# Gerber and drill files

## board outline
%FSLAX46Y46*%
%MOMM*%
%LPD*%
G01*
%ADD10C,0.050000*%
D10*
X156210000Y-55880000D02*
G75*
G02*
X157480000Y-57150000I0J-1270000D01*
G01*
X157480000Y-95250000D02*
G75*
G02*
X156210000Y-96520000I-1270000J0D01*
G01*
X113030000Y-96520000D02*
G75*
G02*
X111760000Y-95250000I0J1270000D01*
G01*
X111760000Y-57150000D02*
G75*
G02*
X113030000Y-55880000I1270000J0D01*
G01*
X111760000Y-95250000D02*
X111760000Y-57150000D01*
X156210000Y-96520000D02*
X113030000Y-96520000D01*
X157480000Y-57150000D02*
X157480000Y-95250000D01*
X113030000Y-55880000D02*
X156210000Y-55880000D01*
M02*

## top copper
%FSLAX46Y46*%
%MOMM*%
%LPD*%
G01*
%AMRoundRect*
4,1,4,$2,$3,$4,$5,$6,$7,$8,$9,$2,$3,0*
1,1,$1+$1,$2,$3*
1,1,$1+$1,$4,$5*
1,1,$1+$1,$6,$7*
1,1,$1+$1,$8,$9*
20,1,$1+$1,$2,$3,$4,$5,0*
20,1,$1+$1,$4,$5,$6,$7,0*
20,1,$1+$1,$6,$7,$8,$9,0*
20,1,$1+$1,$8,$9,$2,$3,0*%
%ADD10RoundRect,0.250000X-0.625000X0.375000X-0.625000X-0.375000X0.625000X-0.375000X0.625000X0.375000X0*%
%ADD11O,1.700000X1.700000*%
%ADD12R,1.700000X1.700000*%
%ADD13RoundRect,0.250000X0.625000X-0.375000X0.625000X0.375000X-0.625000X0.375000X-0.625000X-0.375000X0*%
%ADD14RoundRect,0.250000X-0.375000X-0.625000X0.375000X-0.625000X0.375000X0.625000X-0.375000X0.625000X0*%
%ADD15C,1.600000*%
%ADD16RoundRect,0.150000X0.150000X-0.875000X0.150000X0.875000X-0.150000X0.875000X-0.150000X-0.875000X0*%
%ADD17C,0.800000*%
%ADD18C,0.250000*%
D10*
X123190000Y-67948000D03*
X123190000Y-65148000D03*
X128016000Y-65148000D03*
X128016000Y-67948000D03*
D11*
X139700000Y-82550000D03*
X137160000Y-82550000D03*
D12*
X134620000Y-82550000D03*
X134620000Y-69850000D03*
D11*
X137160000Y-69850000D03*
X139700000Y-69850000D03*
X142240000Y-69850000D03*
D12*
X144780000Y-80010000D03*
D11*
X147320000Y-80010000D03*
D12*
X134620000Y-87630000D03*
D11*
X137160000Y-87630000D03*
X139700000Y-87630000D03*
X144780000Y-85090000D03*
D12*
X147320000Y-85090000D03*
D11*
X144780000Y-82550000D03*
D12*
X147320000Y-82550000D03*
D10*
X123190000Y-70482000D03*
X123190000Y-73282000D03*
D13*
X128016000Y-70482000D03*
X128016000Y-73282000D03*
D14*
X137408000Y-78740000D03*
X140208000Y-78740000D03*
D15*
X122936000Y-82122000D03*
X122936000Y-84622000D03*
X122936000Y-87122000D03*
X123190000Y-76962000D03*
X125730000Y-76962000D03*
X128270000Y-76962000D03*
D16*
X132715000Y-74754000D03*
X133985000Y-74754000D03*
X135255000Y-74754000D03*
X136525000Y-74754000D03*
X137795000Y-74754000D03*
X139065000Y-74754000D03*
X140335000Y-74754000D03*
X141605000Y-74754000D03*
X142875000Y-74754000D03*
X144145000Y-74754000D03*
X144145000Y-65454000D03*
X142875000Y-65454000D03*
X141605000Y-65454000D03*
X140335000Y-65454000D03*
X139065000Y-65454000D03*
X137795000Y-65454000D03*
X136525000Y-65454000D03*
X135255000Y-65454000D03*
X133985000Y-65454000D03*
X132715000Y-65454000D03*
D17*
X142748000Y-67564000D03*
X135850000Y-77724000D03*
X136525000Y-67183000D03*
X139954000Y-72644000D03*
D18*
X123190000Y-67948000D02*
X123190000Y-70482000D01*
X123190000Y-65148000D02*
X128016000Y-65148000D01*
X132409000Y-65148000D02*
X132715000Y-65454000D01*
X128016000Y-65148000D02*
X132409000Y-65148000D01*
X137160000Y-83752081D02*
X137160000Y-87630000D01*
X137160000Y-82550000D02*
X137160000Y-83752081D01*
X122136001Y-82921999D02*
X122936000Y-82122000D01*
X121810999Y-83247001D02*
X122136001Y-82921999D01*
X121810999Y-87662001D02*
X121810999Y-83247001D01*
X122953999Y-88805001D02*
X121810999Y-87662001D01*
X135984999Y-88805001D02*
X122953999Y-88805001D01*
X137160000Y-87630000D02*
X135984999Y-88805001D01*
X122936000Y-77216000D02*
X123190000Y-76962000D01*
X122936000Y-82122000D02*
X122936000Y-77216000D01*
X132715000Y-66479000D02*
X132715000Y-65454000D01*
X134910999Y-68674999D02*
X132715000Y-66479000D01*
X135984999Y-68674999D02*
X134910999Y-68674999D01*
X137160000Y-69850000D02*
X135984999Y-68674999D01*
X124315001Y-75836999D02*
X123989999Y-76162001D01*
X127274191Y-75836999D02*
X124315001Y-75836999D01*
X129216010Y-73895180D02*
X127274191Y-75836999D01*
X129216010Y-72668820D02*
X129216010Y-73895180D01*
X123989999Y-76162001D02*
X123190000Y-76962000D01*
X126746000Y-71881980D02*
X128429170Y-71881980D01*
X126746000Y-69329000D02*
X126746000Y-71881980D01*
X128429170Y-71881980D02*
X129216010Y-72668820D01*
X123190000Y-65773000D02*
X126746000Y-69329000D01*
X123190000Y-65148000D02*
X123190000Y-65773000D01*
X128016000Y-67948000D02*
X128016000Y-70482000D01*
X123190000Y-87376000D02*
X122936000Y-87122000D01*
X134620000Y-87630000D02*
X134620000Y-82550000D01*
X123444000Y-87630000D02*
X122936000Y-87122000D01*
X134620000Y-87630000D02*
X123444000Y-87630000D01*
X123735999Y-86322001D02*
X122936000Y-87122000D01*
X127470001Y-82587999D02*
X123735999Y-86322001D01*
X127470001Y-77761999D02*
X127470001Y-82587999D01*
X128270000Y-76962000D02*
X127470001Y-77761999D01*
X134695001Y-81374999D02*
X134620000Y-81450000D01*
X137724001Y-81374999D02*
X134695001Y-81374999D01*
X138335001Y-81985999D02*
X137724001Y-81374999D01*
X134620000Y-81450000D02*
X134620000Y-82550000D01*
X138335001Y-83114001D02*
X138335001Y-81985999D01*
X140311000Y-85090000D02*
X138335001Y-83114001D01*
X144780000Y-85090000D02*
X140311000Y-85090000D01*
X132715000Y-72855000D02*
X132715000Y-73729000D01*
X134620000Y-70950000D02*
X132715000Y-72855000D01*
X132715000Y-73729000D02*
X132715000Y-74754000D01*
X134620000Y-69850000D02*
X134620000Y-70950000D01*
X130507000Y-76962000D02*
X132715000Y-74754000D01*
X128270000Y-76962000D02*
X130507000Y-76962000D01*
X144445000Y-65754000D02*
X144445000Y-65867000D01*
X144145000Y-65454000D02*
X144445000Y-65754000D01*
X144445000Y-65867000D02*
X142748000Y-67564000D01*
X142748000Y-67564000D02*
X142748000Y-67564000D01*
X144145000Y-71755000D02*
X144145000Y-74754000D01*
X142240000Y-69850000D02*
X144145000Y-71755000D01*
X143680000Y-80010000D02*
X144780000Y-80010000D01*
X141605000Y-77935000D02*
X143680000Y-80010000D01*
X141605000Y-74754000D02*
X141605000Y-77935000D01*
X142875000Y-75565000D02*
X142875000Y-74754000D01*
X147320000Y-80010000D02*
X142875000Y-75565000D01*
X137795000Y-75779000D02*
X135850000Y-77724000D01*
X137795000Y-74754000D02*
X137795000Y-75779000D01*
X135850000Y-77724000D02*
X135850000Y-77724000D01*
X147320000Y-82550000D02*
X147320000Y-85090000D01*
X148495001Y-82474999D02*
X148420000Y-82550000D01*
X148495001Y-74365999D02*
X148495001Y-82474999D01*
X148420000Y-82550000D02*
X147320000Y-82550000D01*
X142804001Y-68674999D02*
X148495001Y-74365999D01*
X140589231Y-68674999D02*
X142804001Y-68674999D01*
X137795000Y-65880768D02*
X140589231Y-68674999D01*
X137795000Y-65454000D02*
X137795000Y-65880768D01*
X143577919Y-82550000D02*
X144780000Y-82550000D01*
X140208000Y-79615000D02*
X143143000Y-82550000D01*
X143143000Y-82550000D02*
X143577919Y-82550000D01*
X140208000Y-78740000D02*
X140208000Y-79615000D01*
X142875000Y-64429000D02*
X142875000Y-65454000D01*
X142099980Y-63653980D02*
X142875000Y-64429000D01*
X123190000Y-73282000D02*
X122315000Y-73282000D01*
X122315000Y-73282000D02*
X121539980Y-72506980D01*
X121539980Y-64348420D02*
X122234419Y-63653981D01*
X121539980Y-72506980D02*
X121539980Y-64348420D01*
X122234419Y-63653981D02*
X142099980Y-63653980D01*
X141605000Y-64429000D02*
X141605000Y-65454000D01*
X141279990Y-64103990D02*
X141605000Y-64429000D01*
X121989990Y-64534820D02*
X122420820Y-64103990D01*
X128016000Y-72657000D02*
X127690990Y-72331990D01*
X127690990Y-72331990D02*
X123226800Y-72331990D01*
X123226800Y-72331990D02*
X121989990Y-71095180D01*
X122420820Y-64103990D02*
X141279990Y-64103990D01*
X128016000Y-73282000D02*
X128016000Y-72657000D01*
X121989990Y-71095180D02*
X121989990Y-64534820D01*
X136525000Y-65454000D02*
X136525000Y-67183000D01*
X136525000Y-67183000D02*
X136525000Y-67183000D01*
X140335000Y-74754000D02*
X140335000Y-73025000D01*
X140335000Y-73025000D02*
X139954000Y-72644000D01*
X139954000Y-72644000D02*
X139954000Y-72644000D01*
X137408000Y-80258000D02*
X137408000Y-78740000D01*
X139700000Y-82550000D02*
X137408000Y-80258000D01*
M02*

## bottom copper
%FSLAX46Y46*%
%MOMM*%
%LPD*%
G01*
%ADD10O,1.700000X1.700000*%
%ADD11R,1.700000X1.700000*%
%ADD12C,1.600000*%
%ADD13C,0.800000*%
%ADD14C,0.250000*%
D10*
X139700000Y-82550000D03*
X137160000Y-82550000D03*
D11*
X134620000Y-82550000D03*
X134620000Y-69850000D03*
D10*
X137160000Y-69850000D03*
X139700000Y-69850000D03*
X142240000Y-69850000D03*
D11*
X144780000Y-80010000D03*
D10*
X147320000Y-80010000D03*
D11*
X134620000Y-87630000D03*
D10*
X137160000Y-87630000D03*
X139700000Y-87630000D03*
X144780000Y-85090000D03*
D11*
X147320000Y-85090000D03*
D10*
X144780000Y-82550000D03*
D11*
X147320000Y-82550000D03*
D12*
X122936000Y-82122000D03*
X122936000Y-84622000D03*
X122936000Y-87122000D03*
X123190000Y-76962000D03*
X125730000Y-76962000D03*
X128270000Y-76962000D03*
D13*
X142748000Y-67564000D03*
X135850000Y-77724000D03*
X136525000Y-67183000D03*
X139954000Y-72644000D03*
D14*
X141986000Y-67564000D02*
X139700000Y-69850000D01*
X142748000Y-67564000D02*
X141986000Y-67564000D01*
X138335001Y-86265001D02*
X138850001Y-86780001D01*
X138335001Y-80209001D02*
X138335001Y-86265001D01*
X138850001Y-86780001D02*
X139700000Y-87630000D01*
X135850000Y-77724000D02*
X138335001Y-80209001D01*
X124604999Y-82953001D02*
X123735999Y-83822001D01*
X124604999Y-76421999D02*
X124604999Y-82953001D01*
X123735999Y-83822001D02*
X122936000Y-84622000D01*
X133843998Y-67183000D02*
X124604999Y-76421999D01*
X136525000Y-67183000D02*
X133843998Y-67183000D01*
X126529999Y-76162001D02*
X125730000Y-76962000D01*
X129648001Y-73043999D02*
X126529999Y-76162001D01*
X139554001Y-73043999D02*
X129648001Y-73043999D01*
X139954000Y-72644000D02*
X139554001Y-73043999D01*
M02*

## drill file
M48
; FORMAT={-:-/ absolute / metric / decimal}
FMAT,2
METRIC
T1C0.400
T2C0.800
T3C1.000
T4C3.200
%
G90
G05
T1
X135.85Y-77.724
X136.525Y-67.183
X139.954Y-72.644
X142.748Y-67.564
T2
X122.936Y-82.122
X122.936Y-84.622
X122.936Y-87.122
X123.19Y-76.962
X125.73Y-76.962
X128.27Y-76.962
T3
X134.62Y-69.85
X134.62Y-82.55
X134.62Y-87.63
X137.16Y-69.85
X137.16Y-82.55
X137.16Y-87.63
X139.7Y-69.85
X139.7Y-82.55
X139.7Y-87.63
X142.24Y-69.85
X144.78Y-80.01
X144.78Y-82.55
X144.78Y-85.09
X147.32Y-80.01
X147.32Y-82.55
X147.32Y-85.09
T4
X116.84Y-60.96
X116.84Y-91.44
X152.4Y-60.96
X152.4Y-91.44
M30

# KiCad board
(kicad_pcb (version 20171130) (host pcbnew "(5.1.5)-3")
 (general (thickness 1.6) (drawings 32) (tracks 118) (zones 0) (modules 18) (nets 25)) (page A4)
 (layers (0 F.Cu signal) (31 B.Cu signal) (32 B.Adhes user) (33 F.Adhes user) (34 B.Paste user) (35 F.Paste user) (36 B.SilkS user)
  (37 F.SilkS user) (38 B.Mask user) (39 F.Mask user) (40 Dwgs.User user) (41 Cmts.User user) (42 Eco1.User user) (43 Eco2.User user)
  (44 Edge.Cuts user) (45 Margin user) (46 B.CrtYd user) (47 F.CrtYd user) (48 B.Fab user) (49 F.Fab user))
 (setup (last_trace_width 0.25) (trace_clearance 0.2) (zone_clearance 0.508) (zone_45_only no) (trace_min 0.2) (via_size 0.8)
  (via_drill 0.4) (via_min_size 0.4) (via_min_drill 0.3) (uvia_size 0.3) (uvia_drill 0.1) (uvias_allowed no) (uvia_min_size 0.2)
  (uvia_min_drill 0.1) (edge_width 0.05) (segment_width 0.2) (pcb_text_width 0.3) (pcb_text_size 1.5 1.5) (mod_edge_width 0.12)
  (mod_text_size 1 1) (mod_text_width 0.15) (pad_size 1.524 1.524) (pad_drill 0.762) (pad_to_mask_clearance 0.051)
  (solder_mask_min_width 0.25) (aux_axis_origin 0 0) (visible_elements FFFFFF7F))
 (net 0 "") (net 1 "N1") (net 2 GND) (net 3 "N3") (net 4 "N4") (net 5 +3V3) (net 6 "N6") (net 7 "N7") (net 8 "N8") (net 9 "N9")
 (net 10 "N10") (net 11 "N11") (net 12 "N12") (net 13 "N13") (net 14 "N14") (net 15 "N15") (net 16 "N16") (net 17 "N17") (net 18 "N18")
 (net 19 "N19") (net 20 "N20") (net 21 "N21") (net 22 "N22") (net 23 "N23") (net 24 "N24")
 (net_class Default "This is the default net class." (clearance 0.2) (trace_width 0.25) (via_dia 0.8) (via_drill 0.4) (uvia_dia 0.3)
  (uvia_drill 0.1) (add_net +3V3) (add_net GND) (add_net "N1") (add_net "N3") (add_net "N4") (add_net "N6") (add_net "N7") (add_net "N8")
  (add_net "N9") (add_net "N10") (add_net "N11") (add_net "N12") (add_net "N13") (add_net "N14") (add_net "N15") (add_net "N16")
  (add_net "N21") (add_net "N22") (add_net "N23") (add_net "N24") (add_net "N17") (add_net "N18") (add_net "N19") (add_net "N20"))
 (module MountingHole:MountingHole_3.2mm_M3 (layer F.Cu) (at 116.84 91.44)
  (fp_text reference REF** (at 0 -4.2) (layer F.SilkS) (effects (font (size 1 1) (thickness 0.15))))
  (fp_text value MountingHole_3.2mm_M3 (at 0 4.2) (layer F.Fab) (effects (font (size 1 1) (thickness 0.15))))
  (pad 1 np_thru_hole circle (at 0 0) (size 3.2 3.2) (drill 3.2) (layers *.Cu *.Mask)))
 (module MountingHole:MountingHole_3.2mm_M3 (layer F.Cu) (at 152.4 91.44)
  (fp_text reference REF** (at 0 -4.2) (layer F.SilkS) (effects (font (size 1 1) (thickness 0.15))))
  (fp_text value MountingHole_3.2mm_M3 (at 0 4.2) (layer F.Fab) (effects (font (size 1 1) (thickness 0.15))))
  (pad 1 np_thru_hole circle (at 0 0) (size 3.2 3.2) (drill 3.2) (layers *.Cu *.Mask)))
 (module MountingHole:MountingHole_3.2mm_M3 (layer F.Cu) (at 152.4 60.96)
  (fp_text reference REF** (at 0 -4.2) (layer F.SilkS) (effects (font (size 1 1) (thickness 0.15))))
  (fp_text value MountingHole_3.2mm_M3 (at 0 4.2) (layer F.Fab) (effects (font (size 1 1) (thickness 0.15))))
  (pad 1 np_thru_hole circle (at 0 0) (size 3.2 3.2) (drill 3.2) (layers *.Cu *.Mask)))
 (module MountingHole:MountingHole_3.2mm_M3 (layer F.Cu) (at 116.84 60.96)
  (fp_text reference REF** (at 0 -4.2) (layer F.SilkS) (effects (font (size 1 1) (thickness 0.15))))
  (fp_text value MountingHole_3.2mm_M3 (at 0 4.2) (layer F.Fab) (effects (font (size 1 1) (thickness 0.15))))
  (pad 1 np_thru_hole circle (at 0 0) (size 3.2 3.2) (drill 3.2) (layers *.Cu *.Mask)))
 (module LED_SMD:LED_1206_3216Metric (layer F.Cu) (at 123.19 66.548 270)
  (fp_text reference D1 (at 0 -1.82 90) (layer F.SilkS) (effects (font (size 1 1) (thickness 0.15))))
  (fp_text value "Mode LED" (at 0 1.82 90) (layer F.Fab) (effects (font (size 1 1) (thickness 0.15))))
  (pad 2 smd roundrect (at 1.4 0 270) (size 1.25 1.75) (layers F.Cu F.Paste F.Mask) (roundrect_rratio 0.2) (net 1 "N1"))
  (pad 1 smd roundrect (at -1.4 0 270) (size 1.25 1.75) (layers F.Cu F.Paste F.Mask) (roundrect_rratio 0.2) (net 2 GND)))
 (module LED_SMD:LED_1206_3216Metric (layer F.Cu) (at 128.016 66.548 270)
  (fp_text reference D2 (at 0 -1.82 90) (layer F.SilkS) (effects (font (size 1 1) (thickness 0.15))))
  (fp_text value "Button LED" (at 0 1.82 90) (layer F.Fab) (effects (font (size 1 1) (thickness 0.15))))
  (pad 1 smd roundrect (at -1.4 0 270) (size 1.25 1.75) (layers F.Cu F.Paste F.Mask) (roundrect_rratio 0.2) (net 2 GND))
  (pad 2 smd roundrect (at 1.4 0 270) (size 1.25 1.75) (layers F.Cu F.Paste F.Mask) (roundrect_rratio 0.2) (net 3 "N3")))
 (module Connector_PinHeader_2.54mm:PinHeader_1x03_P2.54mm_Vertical (layer F.Cu) (at 134.62 82.55 90)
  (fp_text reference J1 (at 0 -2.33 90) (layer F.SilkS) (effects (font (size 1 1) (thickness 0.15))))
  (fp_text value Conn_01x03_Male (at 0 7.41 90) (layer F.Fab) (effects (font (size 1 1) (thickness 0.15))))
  (pad 3 thru_hole oval (at 0 5.08 90) (size 1.7 1.7) (drill 1) (layers *.Cu *.Mask) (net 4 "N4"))
  (pad 2 thru_hole oval (at 0 2.54 90) (size 1.7 1.7) (drill 1) (layers *.Cu *.Mask) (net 2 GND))
  (pad 1 thru_hole rect (at 0 0 90) (size 1.7 1.7) (drill 1) (layers *.Cu *.Mask) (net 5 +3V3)))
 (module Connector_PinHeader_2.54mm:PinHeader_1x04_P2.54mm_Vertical (layer F.Cu) (at 134.62 69.85 90)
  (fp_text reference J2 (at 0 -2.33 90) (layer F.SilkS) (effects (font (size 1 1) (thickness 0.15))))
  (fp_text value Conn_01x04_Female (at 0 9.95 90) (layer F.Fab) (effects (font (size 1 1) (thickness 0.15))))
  (pad 1 thru_hole rect (at 0 0 90) (size 1.7 1.7) (drill 1) (layers *.Cu *.Mask) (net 5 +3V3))
  (pad 2 thru_hole oval (at 0 2.54 90) (size 1.7 1.7) (drill 1) (layers *.Cu *.Mask) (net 2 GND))
  (pad 3 thru_hole oval (at 0 5.08 90) (size 1.7 1.7) (drill 1) (layers *.Cu *.Mask) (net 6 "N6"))
  (pad 4 thru_hole oval (at 0 7.62 90) (size 1.7 1.7) (drill 1) (layers *.Cu *.Mask) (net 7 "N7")))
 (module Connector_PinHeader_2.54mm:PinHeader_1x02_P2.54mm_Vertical (layer F.Cu) (at 144.78 80.01 90)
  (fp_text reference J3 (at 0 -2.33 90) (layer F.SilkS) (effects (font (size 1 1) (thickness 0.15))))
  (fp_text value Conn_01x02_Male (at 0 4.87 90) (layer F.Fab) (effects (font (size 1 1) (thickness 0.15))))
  (pad 1 thru_hole rect (at 0 0 90) (size 1.7 1.7) (drill 1) (layers *.Cu *.Mask) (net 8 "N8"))
  (pad 2 thru_hole oval (at 0 2.54 90) (size 1.7 1.7) (drill 1) (layers *.Cu *.Mask) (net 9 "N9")))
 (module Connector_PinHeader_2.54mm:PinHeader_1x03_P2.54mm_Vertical (layer F.Cu) (at 134.62 87.63 90)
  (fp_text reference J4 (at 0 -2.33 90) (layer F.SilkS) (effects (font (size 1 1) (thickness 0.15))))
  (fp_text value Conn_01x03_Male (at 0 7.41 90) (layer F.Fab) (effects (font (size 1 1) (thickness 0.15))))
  (pad 1 thru_hole rect (at 0 0 90) (size 1.7 1.7) (drill 1) (layers *.Cu *.Mask) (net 5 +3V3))
  (pad 2 thru_hole oval (at 0 2.54 90) (size 1.7 1.7) (drill 1) (layers *.Cu *.Mask) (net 2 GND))
  (pad 3 thru_hole oval (at 0 5.08 90) (size 1.7 1.7) (drill 1) (layers *.Cu *.Mask) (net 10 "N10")))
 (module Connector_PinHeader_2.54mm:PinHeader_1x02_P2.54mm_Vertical (layer F.Cu) (at 147.32 85.09 270)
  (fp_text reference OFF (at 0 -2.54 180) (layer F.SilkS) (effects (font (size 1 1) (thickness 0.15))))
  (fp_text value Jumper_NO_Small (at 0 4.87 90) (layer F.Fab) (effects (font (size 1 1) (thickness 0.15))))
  (pad 2 thru_hole oval (at 0 2.54 270) (size 1.7 1.7) (drill 1) (layers *.Cu *.Mask) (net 5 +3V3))
  (pad 1 thru_hole rect (at 0 0 270) (size 1.7 1.7) (drill 1) (layers *.Cu *.Mask) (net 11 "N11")))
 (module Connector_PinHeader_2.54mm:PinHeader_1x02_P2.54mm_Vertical (layer F.Cu) (at 147.32 82.55 270)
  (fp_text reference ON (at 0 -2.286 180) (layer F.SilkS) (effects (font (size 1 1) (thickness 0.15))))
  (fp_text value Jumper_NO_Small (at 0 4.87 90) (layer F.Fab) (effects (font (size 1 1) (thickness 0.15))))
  (pad 2 thru_hole oval (at 0 2.54 270) (size 1.7 1.7) (drill 1) (layers *.Cu *.Mask) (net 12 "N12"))
  (pad 1 thru_hole rect (at 0 0 270) (size 1.7 1.7) (drill 1) (layers *.Cu *.Mask) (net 11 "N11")))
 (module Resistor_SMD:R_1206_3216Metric (layer F.Cu) (at 123.19 71.882 270)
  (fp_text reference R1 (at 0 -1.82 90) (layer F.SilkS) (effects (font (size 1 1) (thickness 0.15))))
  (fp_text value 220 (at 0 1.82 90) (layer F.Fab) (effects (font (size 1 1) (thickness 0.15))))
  (pad 1 smd roundrect (at -1.4 0 270) (size 1.25 1.75) (layers F.Cu F.Paste F.Mask) (roundrect_rratio 0.2) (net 1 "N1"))
  (pad 2 smd roundrect (at 1.4 0 270) (size 1.25 1.75) (layers F.Cu F.Paste F.Mask) (roundrect_rratio 0.2) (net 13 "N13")))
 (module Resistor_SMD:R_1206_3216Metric (layer F.Cu) (at 128.016 71.882 90)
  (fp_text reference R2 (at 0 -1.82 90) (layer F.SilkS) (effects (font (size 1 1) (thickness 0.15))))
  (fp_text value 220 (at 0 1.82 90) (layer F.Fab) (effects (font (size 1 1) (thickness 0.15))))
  (pad 2 smd roundrect (at 1.4 0 90) (size 1.25 1.75) (layers F.Cu F.Paste F.Mask) (roundrect_rratio 0.2) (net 3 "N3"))
  (pad 1 smd roundrect (at -1.4 0 90) (size 1.25 1.75) (layers F.Cu F.Paste F.Mask) (roundrect_rratio 0.2) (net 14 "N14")))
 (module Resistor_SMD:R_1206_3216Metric (layer F.Cu) (at 138.808 78.74)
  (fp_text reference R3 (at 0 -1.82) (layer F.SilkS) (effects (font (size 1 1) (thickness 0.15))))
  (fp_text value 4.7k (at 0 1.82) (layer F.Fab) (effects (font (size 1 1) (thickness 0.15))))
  (pad 1 smd roundrect (at -1.4 0) (size 1.25 1.75) (layers F.Cu F.Paste F.Mask) (roundrect_rratio 0.2) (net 4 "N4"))
  (pad 2 smd roundrect (at 1.4 0) (size 1.25 1.75) (layers F.Cu F.Paste F.Mask) (roundrect_rratio 0.2) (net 12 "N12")))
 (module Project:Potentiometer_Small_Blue (layer F.Cu) (at 122.936 87.122)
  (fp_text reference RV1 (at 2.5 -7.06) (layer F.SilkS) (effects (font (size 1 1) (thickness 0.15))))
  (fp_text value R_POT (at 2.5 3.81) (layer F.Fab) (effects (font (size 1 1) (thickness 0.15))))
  (pad 3 thru_hole circle (at 0 -5) (size 1.6 1.6) (drill 0.8) (layers *.Cu *.Mask) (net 2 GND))
  (pad 2 thru_hole circle (at 0 -2.5) (size 1.6 1.6) (drill 0.8) (layers *.Cu *.Mask) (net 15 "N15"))
  (pad 1 thru_hole circle (at 0 0) (size 1.6 1.6) (drill 0.8) (layers *.Cu *.Mask) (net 5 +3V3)))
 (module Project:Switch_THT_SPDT (layer F.Cu) (at 125.73 76.962)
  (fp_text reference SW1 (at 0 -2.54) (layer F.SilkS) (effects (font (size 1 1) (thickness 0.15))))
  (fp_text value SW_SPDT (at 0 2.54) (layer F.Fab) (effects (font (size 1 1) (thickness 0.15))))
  (pad 1 thru_hole circle (at -2.54 0) (size 1.6 1.6) (drill 0.8) (layers *.Cu *.Mask) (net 2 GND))
  (pad 2 thru_hole circle (at 0 0) (size 1.6 1.6) (drill 0.8) (layers *.Cu *.Mask) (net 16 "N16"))
  (pad 3 thru_hole circle (at 2.54 0) (size 1.6 1.6) (drill 0.8) (layers *.Cu *.Mask) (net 5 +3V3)))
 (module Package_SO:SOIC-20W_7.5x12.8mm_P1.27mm (layer F.Cu) (at 138.43 70.104 90)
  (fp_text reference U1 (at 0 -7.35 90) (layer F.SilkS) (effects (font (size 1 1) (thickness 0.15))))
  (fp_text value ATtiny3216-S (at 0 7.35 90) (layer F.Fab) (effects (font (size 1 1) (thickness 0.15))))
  (pad 1 smd roundrect (at -4.65 -5.715 90) (size 2.05 0.6) (layers F.Cu F.Paste F.Mask) (roundrect_rratio 0.25) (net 5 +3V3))
  (pad 2 smd roundrect (at -4.65 -4.445 90) (size 2.05 0.6) (layers F.Cu F.Paste F.Mask) (roundrect_rratio 0.25) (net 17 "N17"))
  (pad 3 smd roundrect (at -4.65 -3.175 90) (size 2.05 0.6) (layers F.Cu F.Paste F.Mask) (roundrect_rratio 0.25) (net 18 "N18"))
  (pad 4 smd roundrect (at -4.65 -1.905 90) (size 2.05 0.6) (layers F.Cu F.Paste F.Mask) (roundrect_rratio 0.25) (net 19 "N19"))
  (pad 5 smd roundrect (at -4.65 -0.635 90) (size 2.05 0.6) (layers F.Cu F.Paste F.Mask) (roundrect_rratio 0.25) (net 10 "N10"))
  (pad 6 smd roundrect (at -4.65 0.635 90) (size 2.05 0.6) (layers F.Cu F.Paste F.Mask) (roundrect_rratio 0.25) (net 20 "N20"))
  (pad 7 smd roundrect (at -4.65 1.905 90) (size 2.05 0.6) (layers F.Cu F.Paste F.Mask) (roundrect_rratio 0.25) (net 16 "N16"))
  (pad 8 smd roundrect (at -4.65 3.175 90) (size 2.05 0.6) (layers F.Cu F.Paste F.Mask) (roundrect_rratio 0.25) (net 8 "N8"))
  (pad 9 smd roundrect (at -4.65 4.445 90) (size 2.05 0.6) (layers F.Cu F.Paste F.Mask) (roundrect_rratio 0.25) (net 9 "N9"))
  (pad 10 smd roundrect (at -4.65 5.715 90) (size 2.05 0.6) (layers F.Cu F.Paste F.Mask) (roundrect_rratio 0.25) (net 7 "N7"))
  (pad 11 smd roundrect (at 4.65 5.715 90) (size 2.05 0.6) (layers F.Cu F.Paste F.Mask) (roundrect_rratio 0.25) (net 6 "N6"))
  (pad 12 smd roundrect (at 4.65 4.445 90) (size 2.05 0.6) (layers F.Cu F.Paste F.Mask) (roundrect_rratio 0.25) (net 13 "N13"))
  (pad 13 smd roundrect (at 4.65 3.175 90) (size 2.05 0.6) (layers F.Cu F.Paste F.Mask) (roundrect_rratio 0.25) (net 14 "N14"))
  (pad 14 smd roundrect (at 4.65 1.905 90) (size 2.05 0.6) (layers F.Cu F.Paste F.Mask) (roundrect_rratio 0.25) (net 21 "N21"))
  (pad 15 smd roundrect (at 4.65 0.635 90) (size 2.05 0.6) (layers F.Cu F.Paste F.Mask) (roundrect_rratio 0.25) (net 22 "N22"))
  (pad 16 smd roundrect (at 4.65 -0.635 90) (size 2.05 0.6) (layers F.Cu F.Paste F.Mask) (roundrect_rratio 0.25) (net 11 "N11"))
  (pad 17 smd roundrect (at 4.65 -1.905 90) (size 2.05 0.6) (layers F.Cu F.Paste F.Mask) (roundrect_rratio 0.25) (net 15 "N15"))
  (pad 18 smd roundrect (at 4.65 -3.175 90) (size 2.05 0.6) (layers F.Cu F.Paste F.Mask) (roundrect_rratio 0.25) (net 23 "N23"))
  (pad 19 smd roundrect (at 4.65 -4.445 90) (size 2.05 0.6) (layers F.Cu F.Paste F.Mask) (roundrect_rratio 0.25) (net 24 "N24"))
  (pad 20 smd roundrect (at 4.65 -5.715 90) (size 2.05 0.6) (layers F.Cu F.Paste F.Mask) (roundrect_rratio 0.25) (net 2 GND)))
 (gr_arc (start 156.21 57.15) (end 157.48 57.15) (angle -90) (layer Edge.Cuts) (width 0.05))
 (gr_arc (start 156.21 95.25) (end 156.21 96.52) (angle -90) (layer Edge.Cuts) (width 0.05))
 (gr_arc (start 113.03 95.25) (end 111.76 95.25) (angle -90) (layer Edge.Cuts) (width 0.05))
 (gr_arc (start 113.03 57.15) (end 113.03 55.88) (angle -90) (layer Edge.Cuts) (width 0.05))
 (gr_line (start 111.76 95.25) (end 111.76 57.15) (layer Edge.Cuts) (width 0.05))
 (gr_line (start 156.21 96.52) (end 113.03 96.52) (layer Edge.Cuts) (width 0.05))
 (gr_line (start 157.48 57.15) (end 157.48 95.25) (layer Edge.Cuts) (width 0.05))
 (gr_line (start 113.03 55.88) (end 156.21 55.88) (layer Edge.Cuts) (width 0.05))
 (segment (start 123.19 67.948) (end 123.19 70.482) (width 0.25) (layer F.Cu) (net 1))
 (segment (start 123.19 65.148) (end 128.016 65.148) (width 0.25) (layer F.Cu) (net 2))
 (segment (start 132.409 65.148) (end 132.715 65.454) (width 0.25) (layer F.Cu) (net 2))
 (segment (start 128.016 65.148) (end 132.409 65.148) (width 0.25) (layer F.Cu) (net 2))
 (segment (start 137.16 83.752081) (end 137.16 87.63) (width 0.25) (layer F.Cu) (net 2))
 (segment (start 137.16 82.55) (end 137.16 83.752081) (width 0.25) (layer F.Cu) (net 2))
 (segment (start 122.136001 82.921999) (end 122.936 82.122) (width 0.25) (layer F.Cu) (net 2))
 (segment (start 121.810999 83.247001) (end 122.136001 82.921999) (width 0.25) (layer F.Cu) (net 2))
 (segment (start 121.810999 87.662001) (end 121.810999 83.247001) (width 0.25) (layer F.Cu) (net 2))
 (segment (start 122.953999 88.805001) (end 121.810999 87.662001) (width 0.25) (layer F.Cu) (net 2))
 (segment (start 135.984999 88.805001) (end 122.953999 88.805001) (width 0.25) (layer F.Cu) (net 2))
 (segment (start 137.16 87.63) (end 135.984999 88.805001) (width 0.25) (layer F.Cu) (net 2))
 (segment (start 122.936 77.216) (end 123.19 76.962) (width 0.25) (layer F.Cu) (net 2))
 (segment (start 122.936 82.122) (end 122.936 77.216) (width 0.25) (layer F.Cu) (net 2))
 (segment (start 132.715 66.479) (end 132.715 65.454) (width 0.25) (layer F.Cu) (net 2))
 (segment (start 134.910999 68.674999) (end 132.715 66.479) (width 0.25) (layer F.Cu) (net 2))
 (segment (start 135.984999 68.674999) (end 134.910999 68.674999) (width 0.25) (layer F.Cu) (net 2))
 (segment (start 137.16 69.85) (end 135.984999 68.674999) (width 0.25) (layer F.Cu) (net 2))
 (segment (start 124.315001 75.836999) (end 123.989999 76.162001) (width 0.25) (layer F.Cu) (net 2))
 (segment (start 127.274191 75.836999) (end 124.315001 75.836999) (width 0.25) (layer F.Cu) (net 2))
 (segment (start 129.21601 73.89518) (end 127.274191 75.836999) (width 0.25) (layer F.Cu) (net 2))
 (segment (start 129.21601 72.66882) (end 129.21601 73.89518) (width 0.25) (layer F.Cu) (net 2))
 (segment (start 123.989999 76.162001) (end 123.19 76.962) (width 0.25) (layer F.Cu) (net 2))
 (segment (start 126.746 71.88198) (end 128.42917 71.88198) (width 0.25) (layer F.Cu) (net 2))
 (segment (start 126.746 69.329) (end 126.746 71.88198) (width 0.25) (layer F.Cu) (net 2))
 (segment (start 128.42917 71.88198) (end 129.21601 72.66882) (width 0.25) (layer F.Cu) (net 2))
 (segment (start 123.19 65.773) (end 126.746 69.329) (width 0.25) (layer F.Cu) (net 2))
 (segment (start 123.19 65.148) (end 123.19 65.773) (width 0.25) (layer F.Cu) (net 2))
 (segment (start 128.016 67.948) (end 128.016 70.482) (width 0.25) (layer F.Cu) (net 3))
 (segment (start 123.19 87.376) (end 122.936 87.122) (width 0.25) (layer F.Cu) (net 5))
 (segment (start 134.62 87.63) (end 134.62 82.55) (width 0.25) (layer F.Cu) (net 5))
 (segment (start 123.444 87.63) (end 122.936 87.122) (width 0.25) (layer F.Cu) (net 5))
 (segment (start 134.62 87.63) (end 123.444 87.63) (width 0.25) (layer F.Cu) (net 5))
 (segment (start 123.735999 86.322001) (end 122.936 87.122) (width 0.25) (layer F.Cu) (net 5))
 (segment (start 127.470001 82.587999) (end 123.735999 86.322001) (width 0.25) (layer F.Cu) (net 5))
 (segment (start 127.470001 77.761999) (end 127.470001 82.587999) (width 0.25) (layer F.Cu) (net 5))
 (segment (start 128.27 76.962) (end 127.470001 77.761999) (width 0.25) (layer F.Cu) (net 5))
 (segment (start 134.695001 81.374999) (end 134.62 81.45) (width 0.25) (layer F.Cu) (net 5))
 (segment (start 137.724001 81.374999) (end 134.695001 81.374999) (width 0.25) (layer F.Cu) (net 5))
 (segment (start 138.335001 81.985999) (end 137.724001 81.374999) (width 0.25) (layer F.Cu) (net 5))
 (segment (start 134.62 81.45) (end 134.62 82.55) (width 0.25) (layer F.Cu) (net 5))
 (segment (start 138.335001 83.114001) (end 138.335001 81.985999) (width 0.25) (layer F.Cu) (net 5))
 (segment (start 140.311 85.09) (end 138.335001 83.114001) (width 0.25) (layer F.Cu) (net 5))
 (segment (start 144.78 85.09) (end 140.311 85.09) (width 0.25) (layer F.Cu) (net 5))
 (segment (start 132.715 72.855) (end 132.715 73.729) (width 0.25) (layer F.Cu) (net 5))
 (segment (start 134.62 70.95) (end 132.715 72.855) (width 0.25) (layer F.Cu) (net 5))
 (segment (start 132.715 73.729) (end 132.715 74.754) (width 0.25) (layer F.Cu) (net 5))
 (segment (start 134.62 69.85) (end 134.62 70.95) (width 0.25) (layer F.Cu) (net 5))
 (segment (start 130.507 76.962) (end 132.715 74.754) (width 0.25) (layer F.Cu) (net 5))
 (segment (start 128.27 76.962) (end 130.507 76.962) (width 0.25) (layer F.Cu) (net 5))
 (segment (start 144.445 65.754) (end 144.445 65.867) (width 0.25) (layer F.Cu) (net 6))
 (segment (start 144.145 65.454) (end 144.445 65.754) (width 0.25) (layer F.Cu) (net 6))
 (segment (start 144.445 65.867) (end 142.748 67.564) (width 0.25) (layer F.Cu) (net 6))
 (segment (start 142.748 67.564) (end 142.748 67.564) (width 0.25) (layer F.Cu) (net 6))
 (via (at 142.748 67.564) (size 0.8) (drill 0.4) (layers F.Cu B.Cu) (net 6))
 (segment (start 141.986 67.564) (end 139.7 69.85) (width 0.25) (layer B.Cu) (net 6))
 (segment (start 142.748 67.564) (end 141.986 67.564) (width 0.25) (layer B.Cu) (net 6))
 (segment (start 144.145 71.755) (end 144.145 74.754) (width 0.25) (layer F.Cu) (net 7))
 (segment (start 142.24 69.85) (end 144.145 71.755) (width 0.25) (layer F.Cu) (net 7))
 (segment (start 143.68 80.01) (end 144.78 80.01) (width 0.25) (layer F.Cu) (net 8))
 (segment (start 141.605 77.935) (end 143.68 80.01) (width 0.25) (layer F.Cu) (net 8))
 (segment (start 141.605 74.754) (end 141.605 77.935) (width 0.25) (layer F.Cu) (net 8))
 (segment (start 142.875 75.565) (end 142.875 74.754) (width 0.25) (layer F.Cu) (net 9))
 (segment (start 147.32 80.01) (end 142.875 75.565) (width 0.25) (layer F.Cu) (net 9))
 (segment (start 137.795 75.779) (end 135.85 77.724) (width 0.25) (layer F.Cu) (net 10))
 (segment (start 137.795 74.754) (end 137.795 75.779) (width 0.25) (layer F.Cu) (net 10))
 (segment (start 135.85 77.724) (end 135.85 77.724) (width 0.25) (layer F.Cu) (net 10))
 (via (at 135.85 77.724) (size 0.8) (drill 0.4) (layers F.Cu B.Cu) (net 10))
 (segment (start 138.335001 86.265001) (end 138.850001 86.780001) (width 0.25) (layer B.Cu) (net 10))
 (segment (start 138.335001 80.209001) (end 138.335001 86.265001) (width 0.25) (layer B.Cu) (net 10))
 (segment (start 138.850001 86.780001) (end 139.7 87.63) (width 0.25) (layer B.Cu) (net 10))
 (segment (start 135.85 77.724) (end 138.335001 80.209001) (width 0.25) (layer B.Cu) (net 10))
 (segment (start 147.32 82.55) (end 147.32 85.09) (width 0.25) (layer F.Cu) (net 11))
 (segment (start 148.495001 82.474999) (end 148.42 82.55) (width 0.25) (layer F.Cu) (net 11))
 (segment (start 148.495001 74.365999) (end 148.495001 82.474999) (width 0.25) (layer F.Cu) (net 11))
 (segment (start 148.42 82.55) (end 147.32 82.55) (width 0.25) (layer F.Cu) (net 11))
 (segment (start 142.804001 68.674999) (end 148.495001 74.365999) (width 0.25) (layer F.Cu) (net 11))
 (segment (start 140.589231 68.674999) (end 142.804001 68.674999) (width 0.25) (layer F.Cu) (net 11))
 (segment (start 137.795 65.880768) (end 140.589231 68.674999) (width 0.25) (layer F.Cu) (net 11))
 (segment (start 137.795 65.454) (end 137.795 65.880768) (width 0.25) (layer F.Cu) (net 11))
 (segment (start 143.577919 82.55) (end 144.78 82.55) (width 0.25) (layer F.Cu) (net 12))
 (segment (start 140.208 79.615) (end 143.143 82.55) (width 0.25) (layer F.Cu) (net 12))
 (segment (start 143.143 82.55) (end 143.577919 82.55) (width 0.25) (layer F.Cu) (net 12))
 (segment (start 140.208 78.74) (end 140.208 79.615) (width 0.25) (layer F.Cu) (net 12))
 (segment (start 142.875 64.429) (end 142.875 65.454) (width 0.25) (layer F.Cu) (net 13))
 (segment (start 142.09998 63.65398) (end 142.875 64.429) (width 0.25) (layer F.Cu) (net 13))
 (segment (start 123.19 73.282) (end 122.315 73.282) (width 0.25) (layer F.Cu) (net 13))
 (segment (start 122.315 73.282) (end 121.53998 72.50698) (width 0.25) (layer F.Cu) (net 13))
 (segment (start 121.53998 64.34842) (end 122.234419 63.653981) (width 0.25) (layer F.Cu) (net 13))
 (segment (start 121.53998 72.50698) (end 121.53998 64.34842) (width 0.25) (layer F.Cu) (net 13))
 (segment (start 122.234419 63.653981) (end 142.09998 63.65398) (width 0.25) (layer F.Cu) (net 13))
 (segment (start 141.605 64.429) (end 141.605 65.454) (width 0.25) (layer F.Cu) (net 14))
 (segment (start 141.27999 64.10399) (end 141.605 64.429) (width 0.25) (layer F.Cu) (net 14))
 (segment (start 121.98999 64.53482) (end 122.42082 64.10399) (width 0.25) (layer F.Cu) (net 14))
 (segment (start 128.016 72.657) (end 127.69099 72.33199) (width 0.25) (layer F.Cu) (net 14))
 (segment (start 127.69099 72.33199) (end 123.2268 72.33199) (width 0.25) (layer F.Cu) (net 14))
 (segment (start 123.2268 72.33199) (end 121.98999 71.09518) (width 0.25) (layer F.Cu) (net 14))
 (segment (start 122.42082 64.10399) (end 141.27999 64.10399) (width 0.25) (layer F.Cu) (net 14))
 (segment (start 128.016 73.282) (end 128.016 72.657) (width 0.25) (layer F.Cu) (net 14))
 (segment (start 121.98999 71.09518) (end 121.98999 64.53482) (width 0.25) (layer F.Cu) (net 14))
 (segment (start 136.525 65.454) (end 136.525 67.183) (width 0.25) (layer F.Cu) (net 15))
 (segment (start 136.525 67.183) (end 136.525 67.183) (width 0.25) (layer F.Cu) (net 15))
 (via (at 136.525 67.183) (size 0.8) (drill 0.4) (layers F.Cu B.Cu) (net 15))
 (segment (start 124.604999 82.953001) (end 123.735999 83.822001) (width 0.25) (layer B.Cu) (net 15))
 (segment (start 124.604999 76.421999) (end 124.604999 82.953001) (width 0.25) (layer B.Cu) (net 15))
 (segment (start 123.735999 83.822001) (end 122.936 84.622) (width 0.25) (layer B.Cu) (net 15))
 (segment (start 133.843998 67.183) (end 124.604999 76.421999) (width 0.25) (layer B.Cu) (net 15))
 (segment (start 136.525 67.183) (end 133.843998 67.183) (width 0.25) (layer B.Cu) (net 15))
 (segment (start 140.335 74.754) (end 140.335 73.025) (width 0.25) (layer F.Cu) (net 16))
 (segment (start 140.335 73.025) (end 139.954 72.644) (width 0.25) (layer F.Cu) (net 16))
 (segment (start 139.954 72.644) (end 139.954 72.644) (width 0.25) (layer F.Cu) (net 16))
 (via (at 139.954 72.644) (size 0.8) (drill 0.4) (layers F.Cu B.Cu) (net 16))
 (segment (start 126.529999 76.162001) (end 125.73 76.962) (width 0.25) (layer B.Cu) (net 16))
 (segment (start 129.648001 73.043999) (end 126.529999 76.162001) (width 0.25) (layer B.Cu) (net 16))
 (segment (start 139.554001 73.043999) (end 129.648001 73.043999) (width 0.25) (layer B.Cu) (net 16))
 (segment (start 139.954 72.644) (end 139.554001 73.043999) (width 0.25) (layer B.Cu) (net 16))
 (segment (start 137.408 80.258) (end 137.408 78.74) (width 0.25) (layer F.Cu) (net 4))
 (segment (start 139.7 82.55) (end 137.408 80.258) (width 0.25) (layer F.Cu) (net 4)))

